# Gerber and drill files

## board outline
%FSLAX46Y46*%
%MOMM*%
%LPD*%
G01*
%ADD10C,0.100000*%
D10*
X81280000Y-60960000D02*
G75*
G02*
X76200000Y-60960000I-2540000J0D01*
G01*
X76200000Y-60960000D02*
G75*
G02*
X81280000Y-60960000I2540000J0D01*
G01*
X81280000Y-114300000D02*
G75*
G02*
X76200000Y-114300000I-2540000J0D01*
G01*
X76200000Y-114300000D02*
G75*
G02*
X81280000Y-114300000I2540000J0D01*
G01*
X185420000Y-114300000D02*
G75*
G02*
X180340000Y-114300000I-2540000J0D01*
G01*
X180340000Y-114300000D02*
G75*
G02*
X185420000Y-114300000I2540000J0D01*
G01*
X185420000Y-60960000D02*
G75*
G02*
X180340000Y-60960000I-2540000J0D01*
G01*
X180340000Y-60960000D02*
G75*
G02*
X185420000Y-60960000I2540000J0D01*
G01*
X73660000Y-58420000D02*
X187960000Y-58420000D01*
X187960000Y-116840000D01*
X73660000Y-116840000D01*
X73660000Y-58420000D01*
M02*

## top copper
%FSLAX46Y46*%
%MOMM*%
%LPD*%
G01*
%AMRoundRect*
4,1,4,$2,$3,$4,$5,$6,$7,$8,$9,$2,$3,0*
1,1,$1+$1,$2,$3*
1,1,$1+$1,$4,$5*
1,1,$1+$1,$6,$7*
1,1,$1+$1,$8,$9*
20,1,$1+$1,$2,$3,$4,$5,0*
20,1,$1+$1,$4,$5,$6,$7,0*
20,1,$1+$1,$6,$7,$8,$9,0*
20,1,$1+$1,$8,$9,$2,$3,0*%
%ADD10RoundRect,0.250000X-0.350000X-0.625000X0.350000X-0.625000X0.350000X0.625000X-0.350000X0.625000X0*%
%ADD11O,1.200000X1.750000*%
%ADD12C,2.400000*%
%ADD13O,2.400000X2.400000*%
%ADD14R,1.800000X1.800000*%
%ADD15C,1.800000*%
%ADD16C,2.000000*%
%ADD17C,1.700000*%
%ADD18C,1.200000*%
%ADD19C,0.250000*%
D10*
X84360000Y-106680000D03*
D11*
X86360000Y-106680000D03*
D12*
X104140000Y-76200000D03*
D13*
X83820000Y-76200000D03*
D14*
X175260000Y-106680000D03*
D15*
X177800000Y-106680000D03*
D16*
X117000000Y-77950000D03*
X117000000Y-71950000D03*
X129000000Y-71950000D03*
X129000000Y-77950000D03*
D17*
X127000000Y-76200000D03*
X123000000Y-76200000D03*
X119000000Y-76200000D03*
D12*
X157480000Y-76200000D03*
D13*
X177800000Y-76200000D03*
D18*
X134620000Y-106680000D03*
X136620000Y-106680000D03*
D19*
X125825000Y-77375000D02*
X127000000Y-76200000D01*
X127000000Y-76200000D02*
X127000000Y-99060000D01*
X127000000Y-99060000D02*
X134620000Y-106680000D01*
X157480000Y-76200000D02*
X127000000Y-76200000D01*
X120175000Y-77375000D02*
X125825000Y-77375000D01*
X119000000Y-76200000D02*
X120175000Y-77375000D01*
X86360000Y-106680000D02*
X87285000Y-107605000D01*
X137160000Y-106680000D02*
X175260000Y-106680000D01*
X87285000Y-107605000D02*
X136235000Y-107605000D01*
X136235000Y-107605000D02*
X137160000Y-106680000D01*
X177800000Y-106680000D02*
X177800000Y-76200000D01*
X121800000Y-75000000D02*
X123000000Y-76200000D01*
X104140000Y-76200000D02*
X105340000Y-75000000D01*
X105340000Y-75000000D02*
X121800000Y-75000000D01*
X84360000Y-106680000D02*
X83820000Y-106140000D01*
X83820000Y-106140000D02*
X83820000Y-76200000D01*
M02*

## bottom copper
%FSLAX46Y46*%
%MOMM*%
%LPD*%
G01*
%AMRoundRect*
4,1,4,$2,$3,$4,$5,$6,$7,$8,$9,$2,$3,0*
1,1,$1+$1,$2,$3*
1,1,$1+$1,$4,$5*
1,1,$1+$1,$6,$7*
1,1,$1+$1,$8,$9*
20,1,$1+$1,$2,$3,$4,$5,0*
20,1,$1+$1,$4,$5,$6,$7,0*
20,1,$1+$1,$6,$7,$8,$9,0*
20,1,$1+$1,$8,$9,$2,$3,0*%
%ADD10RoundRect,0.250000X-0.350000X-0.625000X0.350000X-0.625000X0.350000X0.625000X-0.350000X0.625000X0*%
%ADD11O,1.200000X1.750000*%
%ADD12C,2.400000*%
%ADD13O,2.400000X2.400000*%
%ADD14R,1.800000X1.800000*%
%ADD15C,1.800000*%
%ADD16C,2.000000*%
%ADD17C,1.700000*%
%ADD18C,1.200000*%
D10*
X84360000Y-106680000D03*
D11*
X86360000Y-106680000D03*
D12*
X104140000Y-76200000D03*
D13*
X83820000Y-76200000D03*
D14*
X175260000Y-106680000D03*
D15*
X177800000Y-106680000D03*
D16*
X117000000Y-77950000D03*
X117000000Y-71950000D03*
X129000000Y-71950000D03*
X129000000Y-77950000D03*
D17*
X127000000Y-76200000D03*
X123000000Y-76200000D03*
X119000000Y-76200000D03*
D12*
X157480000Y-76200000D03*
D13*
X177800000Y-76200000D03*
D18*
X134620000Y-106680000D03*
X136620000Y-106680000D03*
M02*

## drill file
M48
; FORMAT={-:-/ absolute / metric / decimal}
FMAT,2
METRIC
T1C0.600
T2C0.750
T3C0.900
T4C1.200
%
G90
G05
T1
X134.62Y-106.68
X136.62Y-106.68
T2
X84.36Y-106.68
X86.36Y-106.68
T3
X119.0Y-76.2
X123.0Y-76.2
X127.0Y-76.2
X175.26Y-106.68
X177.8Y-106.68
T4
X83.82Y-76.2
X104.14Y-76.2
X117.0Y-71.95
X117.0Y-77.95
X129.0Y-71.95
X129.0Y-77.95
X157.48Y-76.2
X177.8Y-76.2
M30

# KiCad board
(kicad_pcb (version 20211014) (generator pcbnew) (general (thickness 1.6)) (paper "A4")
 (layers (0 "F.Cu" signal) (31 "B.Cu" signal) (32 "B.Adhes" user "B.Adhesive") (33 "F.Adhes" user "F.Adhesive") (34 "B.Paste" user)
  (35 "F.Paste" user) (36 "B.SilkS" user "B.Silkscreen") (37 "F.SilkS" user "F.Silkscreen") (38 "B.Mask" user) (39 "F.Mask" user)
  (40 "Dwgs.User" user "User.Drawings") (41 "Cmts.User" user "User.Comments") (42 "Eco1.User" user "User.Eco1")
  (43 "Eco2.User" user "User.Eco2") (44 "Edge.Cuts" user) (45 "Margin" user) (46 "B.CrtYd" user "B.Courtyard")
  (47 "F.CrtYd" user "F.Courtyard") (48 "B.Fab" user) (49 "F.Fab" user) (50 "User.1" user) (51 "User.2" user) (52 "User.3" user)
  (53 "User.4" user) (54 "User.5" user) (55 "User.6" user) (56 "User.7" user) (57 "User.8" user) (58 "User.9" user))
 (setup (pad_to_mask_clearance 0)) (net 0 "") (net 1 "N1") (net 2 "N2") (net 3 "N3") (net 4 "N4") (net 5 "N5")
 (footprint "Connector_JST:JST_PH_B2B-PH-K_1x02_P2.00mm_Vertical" (layer "F.Cu") (at 84.36 106.68)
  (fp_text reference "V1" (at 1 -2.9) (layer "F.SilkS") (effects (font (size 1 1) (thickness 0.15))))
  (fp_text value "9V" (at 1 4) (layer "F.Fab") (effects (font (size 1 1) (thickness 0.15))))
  (pad "1" thru_hole roundrect (at 0 0) (size 1.2 1.75) (drill 0.75) (layers *.Cu *.Mask) (roundrect_rratio 0.2083333333) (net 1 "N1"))
  (pad "2" thru_hole oval (at 2 0) (size 1.2 1.75) (drill 0.75) (layers *.Cu *.Mask) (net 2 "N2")))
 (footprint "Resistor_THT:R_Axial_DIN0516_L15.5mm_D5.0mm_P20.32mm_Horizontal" (layer "F.Cu") (at 104.14 76.2 180)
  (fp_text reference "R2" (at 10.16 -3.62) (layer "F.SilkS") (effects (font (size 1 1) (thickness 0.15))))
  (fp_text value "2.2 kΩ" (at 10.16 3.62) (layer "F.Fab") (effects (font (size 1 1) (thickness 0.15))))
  (pad "1" thru_hole circle (at 0 0 180) (size 2.4 2.4) (drill 1.2) (layers *.Cu *.Mask) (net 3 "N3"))
  (pad "2" thru_hole oval (at 20.32 0 180) (size 2.4 2.4) (drill 1.2) (layers *.Cu *.Mask) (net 1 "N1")))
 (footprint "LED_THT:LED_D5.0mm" (layer "F.Cu") (at 175.26 106.68)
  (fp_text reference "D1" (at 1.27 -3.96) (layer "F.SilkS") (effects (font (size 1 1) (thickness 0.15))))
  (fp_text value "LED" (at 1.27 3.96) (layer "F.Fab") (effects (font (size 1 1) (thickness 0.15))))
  (pad "1" thru_hole rect (at 0 0) (size 1.8 1.8) (drill 0.9) (layers *.Cu *.Mask) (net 2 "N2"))
  (pad "2" thru_hole circle (at 2.54 0) (size 1.8 1.8) (drill 0.9) (layers *.Cu *.Mask) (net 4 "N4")))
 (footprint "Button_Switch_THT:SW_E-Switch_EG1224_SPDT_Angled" (layer "F.Cu") (at 127 76.2 180)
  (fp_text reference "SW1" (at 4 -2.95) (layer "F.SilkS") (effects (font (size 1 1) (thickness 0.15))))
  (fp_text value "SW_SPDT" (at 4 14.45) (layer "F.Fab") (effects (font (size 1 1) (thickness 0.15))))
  (pad "" thru_hole circle (at 10 -1.75 180) (size 2 2) (drill 1.2) (layers *.Cu *.Mask))
  (pad "" thru_hole circle (at 10 4.25 180) (size 2 2) (drill 1.2) (layers *.Cu *.Mask))
  (pad "" thru_hole circle (at -2 4.25 180) (size 2 2) (drill 1.2) (layers *.Cu *.Mask))
  (pad "" thru_hole circle (at -2 -1.75 180) (size 2 2) (drill 1.2) (layers *.Cu *.Mask))
  (pad "1" thru_hole circle (at 0 0 180) (size 1.7 1.7) (drill 0.9) (layers *.Cu *.Mask) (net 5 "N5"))
  (pad "2" thru_hole circle (at 4 0 180) (size 1.7 1.7) (drill 0.9) (layers *.Cu *.Mask) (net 3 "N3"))
  (pad "3" thru_hole circle (at 8 0 180) (size 1.7 1.7) (drill 0.9) (layers *.Cu *.Mask) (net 5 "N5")))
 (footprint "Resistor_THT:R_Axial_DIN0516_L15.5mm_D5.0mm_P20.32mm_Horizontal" (layer "F.Cu") (at 157.48 76.2)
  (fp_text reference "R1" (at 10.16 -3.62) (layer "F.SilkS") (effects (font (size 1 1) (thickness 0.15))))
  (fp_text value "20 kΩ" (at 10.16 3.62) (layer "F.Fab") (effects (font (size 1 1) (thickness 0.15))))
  (pad "1" thru_hole circle (at 0 0) (size 2.4 2.4) (drill 1.2) (layers *.Cu *.Mask) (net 5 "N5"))
  (pad "2" thru_hole oval (at 20.32 0) (size 2.4 2.4) (drill 1.2) (layers *.Cu *.Mask) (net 4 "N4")))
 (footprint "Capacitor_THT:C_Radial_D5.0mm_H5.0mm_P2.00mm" (layer "F.Cu") (at 134.62 106.68)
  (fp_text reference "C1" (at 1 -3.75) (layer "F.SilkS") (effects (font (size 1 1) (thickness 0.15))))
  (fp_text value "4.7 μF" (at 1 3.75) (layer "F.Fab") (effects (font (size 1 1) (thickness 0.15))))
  (pad "1" thru_hole circle (at 0 0) (size 1.2 1.2) (drill 0.6) (layers *.Cu *.Mask) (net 5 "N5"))
  (pad "2" thru_hole circle (at 2 0) (size 1.2 1.2) (drill 0.6) (layers *.Cu *.Mask) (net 2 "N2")))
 (gr_circle (center 78.74 60.96) (end 78.74 63.5) (layer "Edge.Cuts") (width 0.1) (fill none))
 (gr_circle (center 78.74 114.3) (end 76.2 114.3) (layer "Edge.Cuts") (width 0.1) (fill none))
 (gr_circle (center 182.88 114.3) (end 182.88 111.76) (layer "Edge.Cuts") (width 0.1) (fill none))
 (gr_circle (center 182.88 60.96) (end 185.42 60.96) (layer "Edge.Cuts") (width 0.1) (fill none))
 (gr_rect (start 187.96 116.84) (end 73.66 58.42) (layer "Edge.Cuts") (width 0.1) (fill none))
 (segment (start 125.825 77.375) (end 127 76.2) (width 0.25) (layer "F.Cu") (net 5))
 (segment (start 127 76.2) (end 127 99.06) (width 0.25) (layer "F.Cu") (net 5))
 (segment (start 127 99.06) (end 134.62 106.68) (width 0.25) (layer "F.Cu") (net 5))
 (segment (start 157.48 76.2) (end 127 76.2) (width 0.25) (layer "F.Cu") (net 5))
 (segment (start 120.175 77.375) (end 125.825 77.375) (width 0.25) (layer "F.Cu") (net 5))
 (segment (start 119 76.2) (end 120.175 77.375) (width 0.25) (layer "F.Cu") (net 5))
 (segment (start 86.36 106.68) (end 87.285 107.605) (width 0.25) (layer "F.Cu") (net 2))
 (segment (start 137.16 106.68) (end 175.26 106.68) (width 0.25) (layer "F.Cu") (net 2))
 (segment (start 87.285 107.605) (end 136.235 107.605) (width 0.25) (layer "F.Cu") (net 2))
 (segment (start 136.235 107.605) (end 137.16 106.68) (width 0.25) (layer "F.Cu") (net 2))
 (segment (start 177.8 106.68) (end 177.8 76.2) (width 0.25) (layer "F.Cu") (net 4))
 (segment (start 121.8 75) (end 123 76.2) (width 0.25) (layer "F.Cu") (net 3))
 (segment (start 104.14 76.2) (end 105.34 75) (width 0.25) (layer "F.Cu") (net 3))
 (segment (start 105.34 75) (end 121.8 75) (width 0.25) (layer "F.Cu") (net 3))
 (segment (start 84.36 106.68) (end 83.82 106.14) (width 0.25) (layer "F.Cu") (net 1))
 (segment (start 83.82 106.14) (end 83.82 76.2) (width 0.25) (layer "F.Cu") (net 1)))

